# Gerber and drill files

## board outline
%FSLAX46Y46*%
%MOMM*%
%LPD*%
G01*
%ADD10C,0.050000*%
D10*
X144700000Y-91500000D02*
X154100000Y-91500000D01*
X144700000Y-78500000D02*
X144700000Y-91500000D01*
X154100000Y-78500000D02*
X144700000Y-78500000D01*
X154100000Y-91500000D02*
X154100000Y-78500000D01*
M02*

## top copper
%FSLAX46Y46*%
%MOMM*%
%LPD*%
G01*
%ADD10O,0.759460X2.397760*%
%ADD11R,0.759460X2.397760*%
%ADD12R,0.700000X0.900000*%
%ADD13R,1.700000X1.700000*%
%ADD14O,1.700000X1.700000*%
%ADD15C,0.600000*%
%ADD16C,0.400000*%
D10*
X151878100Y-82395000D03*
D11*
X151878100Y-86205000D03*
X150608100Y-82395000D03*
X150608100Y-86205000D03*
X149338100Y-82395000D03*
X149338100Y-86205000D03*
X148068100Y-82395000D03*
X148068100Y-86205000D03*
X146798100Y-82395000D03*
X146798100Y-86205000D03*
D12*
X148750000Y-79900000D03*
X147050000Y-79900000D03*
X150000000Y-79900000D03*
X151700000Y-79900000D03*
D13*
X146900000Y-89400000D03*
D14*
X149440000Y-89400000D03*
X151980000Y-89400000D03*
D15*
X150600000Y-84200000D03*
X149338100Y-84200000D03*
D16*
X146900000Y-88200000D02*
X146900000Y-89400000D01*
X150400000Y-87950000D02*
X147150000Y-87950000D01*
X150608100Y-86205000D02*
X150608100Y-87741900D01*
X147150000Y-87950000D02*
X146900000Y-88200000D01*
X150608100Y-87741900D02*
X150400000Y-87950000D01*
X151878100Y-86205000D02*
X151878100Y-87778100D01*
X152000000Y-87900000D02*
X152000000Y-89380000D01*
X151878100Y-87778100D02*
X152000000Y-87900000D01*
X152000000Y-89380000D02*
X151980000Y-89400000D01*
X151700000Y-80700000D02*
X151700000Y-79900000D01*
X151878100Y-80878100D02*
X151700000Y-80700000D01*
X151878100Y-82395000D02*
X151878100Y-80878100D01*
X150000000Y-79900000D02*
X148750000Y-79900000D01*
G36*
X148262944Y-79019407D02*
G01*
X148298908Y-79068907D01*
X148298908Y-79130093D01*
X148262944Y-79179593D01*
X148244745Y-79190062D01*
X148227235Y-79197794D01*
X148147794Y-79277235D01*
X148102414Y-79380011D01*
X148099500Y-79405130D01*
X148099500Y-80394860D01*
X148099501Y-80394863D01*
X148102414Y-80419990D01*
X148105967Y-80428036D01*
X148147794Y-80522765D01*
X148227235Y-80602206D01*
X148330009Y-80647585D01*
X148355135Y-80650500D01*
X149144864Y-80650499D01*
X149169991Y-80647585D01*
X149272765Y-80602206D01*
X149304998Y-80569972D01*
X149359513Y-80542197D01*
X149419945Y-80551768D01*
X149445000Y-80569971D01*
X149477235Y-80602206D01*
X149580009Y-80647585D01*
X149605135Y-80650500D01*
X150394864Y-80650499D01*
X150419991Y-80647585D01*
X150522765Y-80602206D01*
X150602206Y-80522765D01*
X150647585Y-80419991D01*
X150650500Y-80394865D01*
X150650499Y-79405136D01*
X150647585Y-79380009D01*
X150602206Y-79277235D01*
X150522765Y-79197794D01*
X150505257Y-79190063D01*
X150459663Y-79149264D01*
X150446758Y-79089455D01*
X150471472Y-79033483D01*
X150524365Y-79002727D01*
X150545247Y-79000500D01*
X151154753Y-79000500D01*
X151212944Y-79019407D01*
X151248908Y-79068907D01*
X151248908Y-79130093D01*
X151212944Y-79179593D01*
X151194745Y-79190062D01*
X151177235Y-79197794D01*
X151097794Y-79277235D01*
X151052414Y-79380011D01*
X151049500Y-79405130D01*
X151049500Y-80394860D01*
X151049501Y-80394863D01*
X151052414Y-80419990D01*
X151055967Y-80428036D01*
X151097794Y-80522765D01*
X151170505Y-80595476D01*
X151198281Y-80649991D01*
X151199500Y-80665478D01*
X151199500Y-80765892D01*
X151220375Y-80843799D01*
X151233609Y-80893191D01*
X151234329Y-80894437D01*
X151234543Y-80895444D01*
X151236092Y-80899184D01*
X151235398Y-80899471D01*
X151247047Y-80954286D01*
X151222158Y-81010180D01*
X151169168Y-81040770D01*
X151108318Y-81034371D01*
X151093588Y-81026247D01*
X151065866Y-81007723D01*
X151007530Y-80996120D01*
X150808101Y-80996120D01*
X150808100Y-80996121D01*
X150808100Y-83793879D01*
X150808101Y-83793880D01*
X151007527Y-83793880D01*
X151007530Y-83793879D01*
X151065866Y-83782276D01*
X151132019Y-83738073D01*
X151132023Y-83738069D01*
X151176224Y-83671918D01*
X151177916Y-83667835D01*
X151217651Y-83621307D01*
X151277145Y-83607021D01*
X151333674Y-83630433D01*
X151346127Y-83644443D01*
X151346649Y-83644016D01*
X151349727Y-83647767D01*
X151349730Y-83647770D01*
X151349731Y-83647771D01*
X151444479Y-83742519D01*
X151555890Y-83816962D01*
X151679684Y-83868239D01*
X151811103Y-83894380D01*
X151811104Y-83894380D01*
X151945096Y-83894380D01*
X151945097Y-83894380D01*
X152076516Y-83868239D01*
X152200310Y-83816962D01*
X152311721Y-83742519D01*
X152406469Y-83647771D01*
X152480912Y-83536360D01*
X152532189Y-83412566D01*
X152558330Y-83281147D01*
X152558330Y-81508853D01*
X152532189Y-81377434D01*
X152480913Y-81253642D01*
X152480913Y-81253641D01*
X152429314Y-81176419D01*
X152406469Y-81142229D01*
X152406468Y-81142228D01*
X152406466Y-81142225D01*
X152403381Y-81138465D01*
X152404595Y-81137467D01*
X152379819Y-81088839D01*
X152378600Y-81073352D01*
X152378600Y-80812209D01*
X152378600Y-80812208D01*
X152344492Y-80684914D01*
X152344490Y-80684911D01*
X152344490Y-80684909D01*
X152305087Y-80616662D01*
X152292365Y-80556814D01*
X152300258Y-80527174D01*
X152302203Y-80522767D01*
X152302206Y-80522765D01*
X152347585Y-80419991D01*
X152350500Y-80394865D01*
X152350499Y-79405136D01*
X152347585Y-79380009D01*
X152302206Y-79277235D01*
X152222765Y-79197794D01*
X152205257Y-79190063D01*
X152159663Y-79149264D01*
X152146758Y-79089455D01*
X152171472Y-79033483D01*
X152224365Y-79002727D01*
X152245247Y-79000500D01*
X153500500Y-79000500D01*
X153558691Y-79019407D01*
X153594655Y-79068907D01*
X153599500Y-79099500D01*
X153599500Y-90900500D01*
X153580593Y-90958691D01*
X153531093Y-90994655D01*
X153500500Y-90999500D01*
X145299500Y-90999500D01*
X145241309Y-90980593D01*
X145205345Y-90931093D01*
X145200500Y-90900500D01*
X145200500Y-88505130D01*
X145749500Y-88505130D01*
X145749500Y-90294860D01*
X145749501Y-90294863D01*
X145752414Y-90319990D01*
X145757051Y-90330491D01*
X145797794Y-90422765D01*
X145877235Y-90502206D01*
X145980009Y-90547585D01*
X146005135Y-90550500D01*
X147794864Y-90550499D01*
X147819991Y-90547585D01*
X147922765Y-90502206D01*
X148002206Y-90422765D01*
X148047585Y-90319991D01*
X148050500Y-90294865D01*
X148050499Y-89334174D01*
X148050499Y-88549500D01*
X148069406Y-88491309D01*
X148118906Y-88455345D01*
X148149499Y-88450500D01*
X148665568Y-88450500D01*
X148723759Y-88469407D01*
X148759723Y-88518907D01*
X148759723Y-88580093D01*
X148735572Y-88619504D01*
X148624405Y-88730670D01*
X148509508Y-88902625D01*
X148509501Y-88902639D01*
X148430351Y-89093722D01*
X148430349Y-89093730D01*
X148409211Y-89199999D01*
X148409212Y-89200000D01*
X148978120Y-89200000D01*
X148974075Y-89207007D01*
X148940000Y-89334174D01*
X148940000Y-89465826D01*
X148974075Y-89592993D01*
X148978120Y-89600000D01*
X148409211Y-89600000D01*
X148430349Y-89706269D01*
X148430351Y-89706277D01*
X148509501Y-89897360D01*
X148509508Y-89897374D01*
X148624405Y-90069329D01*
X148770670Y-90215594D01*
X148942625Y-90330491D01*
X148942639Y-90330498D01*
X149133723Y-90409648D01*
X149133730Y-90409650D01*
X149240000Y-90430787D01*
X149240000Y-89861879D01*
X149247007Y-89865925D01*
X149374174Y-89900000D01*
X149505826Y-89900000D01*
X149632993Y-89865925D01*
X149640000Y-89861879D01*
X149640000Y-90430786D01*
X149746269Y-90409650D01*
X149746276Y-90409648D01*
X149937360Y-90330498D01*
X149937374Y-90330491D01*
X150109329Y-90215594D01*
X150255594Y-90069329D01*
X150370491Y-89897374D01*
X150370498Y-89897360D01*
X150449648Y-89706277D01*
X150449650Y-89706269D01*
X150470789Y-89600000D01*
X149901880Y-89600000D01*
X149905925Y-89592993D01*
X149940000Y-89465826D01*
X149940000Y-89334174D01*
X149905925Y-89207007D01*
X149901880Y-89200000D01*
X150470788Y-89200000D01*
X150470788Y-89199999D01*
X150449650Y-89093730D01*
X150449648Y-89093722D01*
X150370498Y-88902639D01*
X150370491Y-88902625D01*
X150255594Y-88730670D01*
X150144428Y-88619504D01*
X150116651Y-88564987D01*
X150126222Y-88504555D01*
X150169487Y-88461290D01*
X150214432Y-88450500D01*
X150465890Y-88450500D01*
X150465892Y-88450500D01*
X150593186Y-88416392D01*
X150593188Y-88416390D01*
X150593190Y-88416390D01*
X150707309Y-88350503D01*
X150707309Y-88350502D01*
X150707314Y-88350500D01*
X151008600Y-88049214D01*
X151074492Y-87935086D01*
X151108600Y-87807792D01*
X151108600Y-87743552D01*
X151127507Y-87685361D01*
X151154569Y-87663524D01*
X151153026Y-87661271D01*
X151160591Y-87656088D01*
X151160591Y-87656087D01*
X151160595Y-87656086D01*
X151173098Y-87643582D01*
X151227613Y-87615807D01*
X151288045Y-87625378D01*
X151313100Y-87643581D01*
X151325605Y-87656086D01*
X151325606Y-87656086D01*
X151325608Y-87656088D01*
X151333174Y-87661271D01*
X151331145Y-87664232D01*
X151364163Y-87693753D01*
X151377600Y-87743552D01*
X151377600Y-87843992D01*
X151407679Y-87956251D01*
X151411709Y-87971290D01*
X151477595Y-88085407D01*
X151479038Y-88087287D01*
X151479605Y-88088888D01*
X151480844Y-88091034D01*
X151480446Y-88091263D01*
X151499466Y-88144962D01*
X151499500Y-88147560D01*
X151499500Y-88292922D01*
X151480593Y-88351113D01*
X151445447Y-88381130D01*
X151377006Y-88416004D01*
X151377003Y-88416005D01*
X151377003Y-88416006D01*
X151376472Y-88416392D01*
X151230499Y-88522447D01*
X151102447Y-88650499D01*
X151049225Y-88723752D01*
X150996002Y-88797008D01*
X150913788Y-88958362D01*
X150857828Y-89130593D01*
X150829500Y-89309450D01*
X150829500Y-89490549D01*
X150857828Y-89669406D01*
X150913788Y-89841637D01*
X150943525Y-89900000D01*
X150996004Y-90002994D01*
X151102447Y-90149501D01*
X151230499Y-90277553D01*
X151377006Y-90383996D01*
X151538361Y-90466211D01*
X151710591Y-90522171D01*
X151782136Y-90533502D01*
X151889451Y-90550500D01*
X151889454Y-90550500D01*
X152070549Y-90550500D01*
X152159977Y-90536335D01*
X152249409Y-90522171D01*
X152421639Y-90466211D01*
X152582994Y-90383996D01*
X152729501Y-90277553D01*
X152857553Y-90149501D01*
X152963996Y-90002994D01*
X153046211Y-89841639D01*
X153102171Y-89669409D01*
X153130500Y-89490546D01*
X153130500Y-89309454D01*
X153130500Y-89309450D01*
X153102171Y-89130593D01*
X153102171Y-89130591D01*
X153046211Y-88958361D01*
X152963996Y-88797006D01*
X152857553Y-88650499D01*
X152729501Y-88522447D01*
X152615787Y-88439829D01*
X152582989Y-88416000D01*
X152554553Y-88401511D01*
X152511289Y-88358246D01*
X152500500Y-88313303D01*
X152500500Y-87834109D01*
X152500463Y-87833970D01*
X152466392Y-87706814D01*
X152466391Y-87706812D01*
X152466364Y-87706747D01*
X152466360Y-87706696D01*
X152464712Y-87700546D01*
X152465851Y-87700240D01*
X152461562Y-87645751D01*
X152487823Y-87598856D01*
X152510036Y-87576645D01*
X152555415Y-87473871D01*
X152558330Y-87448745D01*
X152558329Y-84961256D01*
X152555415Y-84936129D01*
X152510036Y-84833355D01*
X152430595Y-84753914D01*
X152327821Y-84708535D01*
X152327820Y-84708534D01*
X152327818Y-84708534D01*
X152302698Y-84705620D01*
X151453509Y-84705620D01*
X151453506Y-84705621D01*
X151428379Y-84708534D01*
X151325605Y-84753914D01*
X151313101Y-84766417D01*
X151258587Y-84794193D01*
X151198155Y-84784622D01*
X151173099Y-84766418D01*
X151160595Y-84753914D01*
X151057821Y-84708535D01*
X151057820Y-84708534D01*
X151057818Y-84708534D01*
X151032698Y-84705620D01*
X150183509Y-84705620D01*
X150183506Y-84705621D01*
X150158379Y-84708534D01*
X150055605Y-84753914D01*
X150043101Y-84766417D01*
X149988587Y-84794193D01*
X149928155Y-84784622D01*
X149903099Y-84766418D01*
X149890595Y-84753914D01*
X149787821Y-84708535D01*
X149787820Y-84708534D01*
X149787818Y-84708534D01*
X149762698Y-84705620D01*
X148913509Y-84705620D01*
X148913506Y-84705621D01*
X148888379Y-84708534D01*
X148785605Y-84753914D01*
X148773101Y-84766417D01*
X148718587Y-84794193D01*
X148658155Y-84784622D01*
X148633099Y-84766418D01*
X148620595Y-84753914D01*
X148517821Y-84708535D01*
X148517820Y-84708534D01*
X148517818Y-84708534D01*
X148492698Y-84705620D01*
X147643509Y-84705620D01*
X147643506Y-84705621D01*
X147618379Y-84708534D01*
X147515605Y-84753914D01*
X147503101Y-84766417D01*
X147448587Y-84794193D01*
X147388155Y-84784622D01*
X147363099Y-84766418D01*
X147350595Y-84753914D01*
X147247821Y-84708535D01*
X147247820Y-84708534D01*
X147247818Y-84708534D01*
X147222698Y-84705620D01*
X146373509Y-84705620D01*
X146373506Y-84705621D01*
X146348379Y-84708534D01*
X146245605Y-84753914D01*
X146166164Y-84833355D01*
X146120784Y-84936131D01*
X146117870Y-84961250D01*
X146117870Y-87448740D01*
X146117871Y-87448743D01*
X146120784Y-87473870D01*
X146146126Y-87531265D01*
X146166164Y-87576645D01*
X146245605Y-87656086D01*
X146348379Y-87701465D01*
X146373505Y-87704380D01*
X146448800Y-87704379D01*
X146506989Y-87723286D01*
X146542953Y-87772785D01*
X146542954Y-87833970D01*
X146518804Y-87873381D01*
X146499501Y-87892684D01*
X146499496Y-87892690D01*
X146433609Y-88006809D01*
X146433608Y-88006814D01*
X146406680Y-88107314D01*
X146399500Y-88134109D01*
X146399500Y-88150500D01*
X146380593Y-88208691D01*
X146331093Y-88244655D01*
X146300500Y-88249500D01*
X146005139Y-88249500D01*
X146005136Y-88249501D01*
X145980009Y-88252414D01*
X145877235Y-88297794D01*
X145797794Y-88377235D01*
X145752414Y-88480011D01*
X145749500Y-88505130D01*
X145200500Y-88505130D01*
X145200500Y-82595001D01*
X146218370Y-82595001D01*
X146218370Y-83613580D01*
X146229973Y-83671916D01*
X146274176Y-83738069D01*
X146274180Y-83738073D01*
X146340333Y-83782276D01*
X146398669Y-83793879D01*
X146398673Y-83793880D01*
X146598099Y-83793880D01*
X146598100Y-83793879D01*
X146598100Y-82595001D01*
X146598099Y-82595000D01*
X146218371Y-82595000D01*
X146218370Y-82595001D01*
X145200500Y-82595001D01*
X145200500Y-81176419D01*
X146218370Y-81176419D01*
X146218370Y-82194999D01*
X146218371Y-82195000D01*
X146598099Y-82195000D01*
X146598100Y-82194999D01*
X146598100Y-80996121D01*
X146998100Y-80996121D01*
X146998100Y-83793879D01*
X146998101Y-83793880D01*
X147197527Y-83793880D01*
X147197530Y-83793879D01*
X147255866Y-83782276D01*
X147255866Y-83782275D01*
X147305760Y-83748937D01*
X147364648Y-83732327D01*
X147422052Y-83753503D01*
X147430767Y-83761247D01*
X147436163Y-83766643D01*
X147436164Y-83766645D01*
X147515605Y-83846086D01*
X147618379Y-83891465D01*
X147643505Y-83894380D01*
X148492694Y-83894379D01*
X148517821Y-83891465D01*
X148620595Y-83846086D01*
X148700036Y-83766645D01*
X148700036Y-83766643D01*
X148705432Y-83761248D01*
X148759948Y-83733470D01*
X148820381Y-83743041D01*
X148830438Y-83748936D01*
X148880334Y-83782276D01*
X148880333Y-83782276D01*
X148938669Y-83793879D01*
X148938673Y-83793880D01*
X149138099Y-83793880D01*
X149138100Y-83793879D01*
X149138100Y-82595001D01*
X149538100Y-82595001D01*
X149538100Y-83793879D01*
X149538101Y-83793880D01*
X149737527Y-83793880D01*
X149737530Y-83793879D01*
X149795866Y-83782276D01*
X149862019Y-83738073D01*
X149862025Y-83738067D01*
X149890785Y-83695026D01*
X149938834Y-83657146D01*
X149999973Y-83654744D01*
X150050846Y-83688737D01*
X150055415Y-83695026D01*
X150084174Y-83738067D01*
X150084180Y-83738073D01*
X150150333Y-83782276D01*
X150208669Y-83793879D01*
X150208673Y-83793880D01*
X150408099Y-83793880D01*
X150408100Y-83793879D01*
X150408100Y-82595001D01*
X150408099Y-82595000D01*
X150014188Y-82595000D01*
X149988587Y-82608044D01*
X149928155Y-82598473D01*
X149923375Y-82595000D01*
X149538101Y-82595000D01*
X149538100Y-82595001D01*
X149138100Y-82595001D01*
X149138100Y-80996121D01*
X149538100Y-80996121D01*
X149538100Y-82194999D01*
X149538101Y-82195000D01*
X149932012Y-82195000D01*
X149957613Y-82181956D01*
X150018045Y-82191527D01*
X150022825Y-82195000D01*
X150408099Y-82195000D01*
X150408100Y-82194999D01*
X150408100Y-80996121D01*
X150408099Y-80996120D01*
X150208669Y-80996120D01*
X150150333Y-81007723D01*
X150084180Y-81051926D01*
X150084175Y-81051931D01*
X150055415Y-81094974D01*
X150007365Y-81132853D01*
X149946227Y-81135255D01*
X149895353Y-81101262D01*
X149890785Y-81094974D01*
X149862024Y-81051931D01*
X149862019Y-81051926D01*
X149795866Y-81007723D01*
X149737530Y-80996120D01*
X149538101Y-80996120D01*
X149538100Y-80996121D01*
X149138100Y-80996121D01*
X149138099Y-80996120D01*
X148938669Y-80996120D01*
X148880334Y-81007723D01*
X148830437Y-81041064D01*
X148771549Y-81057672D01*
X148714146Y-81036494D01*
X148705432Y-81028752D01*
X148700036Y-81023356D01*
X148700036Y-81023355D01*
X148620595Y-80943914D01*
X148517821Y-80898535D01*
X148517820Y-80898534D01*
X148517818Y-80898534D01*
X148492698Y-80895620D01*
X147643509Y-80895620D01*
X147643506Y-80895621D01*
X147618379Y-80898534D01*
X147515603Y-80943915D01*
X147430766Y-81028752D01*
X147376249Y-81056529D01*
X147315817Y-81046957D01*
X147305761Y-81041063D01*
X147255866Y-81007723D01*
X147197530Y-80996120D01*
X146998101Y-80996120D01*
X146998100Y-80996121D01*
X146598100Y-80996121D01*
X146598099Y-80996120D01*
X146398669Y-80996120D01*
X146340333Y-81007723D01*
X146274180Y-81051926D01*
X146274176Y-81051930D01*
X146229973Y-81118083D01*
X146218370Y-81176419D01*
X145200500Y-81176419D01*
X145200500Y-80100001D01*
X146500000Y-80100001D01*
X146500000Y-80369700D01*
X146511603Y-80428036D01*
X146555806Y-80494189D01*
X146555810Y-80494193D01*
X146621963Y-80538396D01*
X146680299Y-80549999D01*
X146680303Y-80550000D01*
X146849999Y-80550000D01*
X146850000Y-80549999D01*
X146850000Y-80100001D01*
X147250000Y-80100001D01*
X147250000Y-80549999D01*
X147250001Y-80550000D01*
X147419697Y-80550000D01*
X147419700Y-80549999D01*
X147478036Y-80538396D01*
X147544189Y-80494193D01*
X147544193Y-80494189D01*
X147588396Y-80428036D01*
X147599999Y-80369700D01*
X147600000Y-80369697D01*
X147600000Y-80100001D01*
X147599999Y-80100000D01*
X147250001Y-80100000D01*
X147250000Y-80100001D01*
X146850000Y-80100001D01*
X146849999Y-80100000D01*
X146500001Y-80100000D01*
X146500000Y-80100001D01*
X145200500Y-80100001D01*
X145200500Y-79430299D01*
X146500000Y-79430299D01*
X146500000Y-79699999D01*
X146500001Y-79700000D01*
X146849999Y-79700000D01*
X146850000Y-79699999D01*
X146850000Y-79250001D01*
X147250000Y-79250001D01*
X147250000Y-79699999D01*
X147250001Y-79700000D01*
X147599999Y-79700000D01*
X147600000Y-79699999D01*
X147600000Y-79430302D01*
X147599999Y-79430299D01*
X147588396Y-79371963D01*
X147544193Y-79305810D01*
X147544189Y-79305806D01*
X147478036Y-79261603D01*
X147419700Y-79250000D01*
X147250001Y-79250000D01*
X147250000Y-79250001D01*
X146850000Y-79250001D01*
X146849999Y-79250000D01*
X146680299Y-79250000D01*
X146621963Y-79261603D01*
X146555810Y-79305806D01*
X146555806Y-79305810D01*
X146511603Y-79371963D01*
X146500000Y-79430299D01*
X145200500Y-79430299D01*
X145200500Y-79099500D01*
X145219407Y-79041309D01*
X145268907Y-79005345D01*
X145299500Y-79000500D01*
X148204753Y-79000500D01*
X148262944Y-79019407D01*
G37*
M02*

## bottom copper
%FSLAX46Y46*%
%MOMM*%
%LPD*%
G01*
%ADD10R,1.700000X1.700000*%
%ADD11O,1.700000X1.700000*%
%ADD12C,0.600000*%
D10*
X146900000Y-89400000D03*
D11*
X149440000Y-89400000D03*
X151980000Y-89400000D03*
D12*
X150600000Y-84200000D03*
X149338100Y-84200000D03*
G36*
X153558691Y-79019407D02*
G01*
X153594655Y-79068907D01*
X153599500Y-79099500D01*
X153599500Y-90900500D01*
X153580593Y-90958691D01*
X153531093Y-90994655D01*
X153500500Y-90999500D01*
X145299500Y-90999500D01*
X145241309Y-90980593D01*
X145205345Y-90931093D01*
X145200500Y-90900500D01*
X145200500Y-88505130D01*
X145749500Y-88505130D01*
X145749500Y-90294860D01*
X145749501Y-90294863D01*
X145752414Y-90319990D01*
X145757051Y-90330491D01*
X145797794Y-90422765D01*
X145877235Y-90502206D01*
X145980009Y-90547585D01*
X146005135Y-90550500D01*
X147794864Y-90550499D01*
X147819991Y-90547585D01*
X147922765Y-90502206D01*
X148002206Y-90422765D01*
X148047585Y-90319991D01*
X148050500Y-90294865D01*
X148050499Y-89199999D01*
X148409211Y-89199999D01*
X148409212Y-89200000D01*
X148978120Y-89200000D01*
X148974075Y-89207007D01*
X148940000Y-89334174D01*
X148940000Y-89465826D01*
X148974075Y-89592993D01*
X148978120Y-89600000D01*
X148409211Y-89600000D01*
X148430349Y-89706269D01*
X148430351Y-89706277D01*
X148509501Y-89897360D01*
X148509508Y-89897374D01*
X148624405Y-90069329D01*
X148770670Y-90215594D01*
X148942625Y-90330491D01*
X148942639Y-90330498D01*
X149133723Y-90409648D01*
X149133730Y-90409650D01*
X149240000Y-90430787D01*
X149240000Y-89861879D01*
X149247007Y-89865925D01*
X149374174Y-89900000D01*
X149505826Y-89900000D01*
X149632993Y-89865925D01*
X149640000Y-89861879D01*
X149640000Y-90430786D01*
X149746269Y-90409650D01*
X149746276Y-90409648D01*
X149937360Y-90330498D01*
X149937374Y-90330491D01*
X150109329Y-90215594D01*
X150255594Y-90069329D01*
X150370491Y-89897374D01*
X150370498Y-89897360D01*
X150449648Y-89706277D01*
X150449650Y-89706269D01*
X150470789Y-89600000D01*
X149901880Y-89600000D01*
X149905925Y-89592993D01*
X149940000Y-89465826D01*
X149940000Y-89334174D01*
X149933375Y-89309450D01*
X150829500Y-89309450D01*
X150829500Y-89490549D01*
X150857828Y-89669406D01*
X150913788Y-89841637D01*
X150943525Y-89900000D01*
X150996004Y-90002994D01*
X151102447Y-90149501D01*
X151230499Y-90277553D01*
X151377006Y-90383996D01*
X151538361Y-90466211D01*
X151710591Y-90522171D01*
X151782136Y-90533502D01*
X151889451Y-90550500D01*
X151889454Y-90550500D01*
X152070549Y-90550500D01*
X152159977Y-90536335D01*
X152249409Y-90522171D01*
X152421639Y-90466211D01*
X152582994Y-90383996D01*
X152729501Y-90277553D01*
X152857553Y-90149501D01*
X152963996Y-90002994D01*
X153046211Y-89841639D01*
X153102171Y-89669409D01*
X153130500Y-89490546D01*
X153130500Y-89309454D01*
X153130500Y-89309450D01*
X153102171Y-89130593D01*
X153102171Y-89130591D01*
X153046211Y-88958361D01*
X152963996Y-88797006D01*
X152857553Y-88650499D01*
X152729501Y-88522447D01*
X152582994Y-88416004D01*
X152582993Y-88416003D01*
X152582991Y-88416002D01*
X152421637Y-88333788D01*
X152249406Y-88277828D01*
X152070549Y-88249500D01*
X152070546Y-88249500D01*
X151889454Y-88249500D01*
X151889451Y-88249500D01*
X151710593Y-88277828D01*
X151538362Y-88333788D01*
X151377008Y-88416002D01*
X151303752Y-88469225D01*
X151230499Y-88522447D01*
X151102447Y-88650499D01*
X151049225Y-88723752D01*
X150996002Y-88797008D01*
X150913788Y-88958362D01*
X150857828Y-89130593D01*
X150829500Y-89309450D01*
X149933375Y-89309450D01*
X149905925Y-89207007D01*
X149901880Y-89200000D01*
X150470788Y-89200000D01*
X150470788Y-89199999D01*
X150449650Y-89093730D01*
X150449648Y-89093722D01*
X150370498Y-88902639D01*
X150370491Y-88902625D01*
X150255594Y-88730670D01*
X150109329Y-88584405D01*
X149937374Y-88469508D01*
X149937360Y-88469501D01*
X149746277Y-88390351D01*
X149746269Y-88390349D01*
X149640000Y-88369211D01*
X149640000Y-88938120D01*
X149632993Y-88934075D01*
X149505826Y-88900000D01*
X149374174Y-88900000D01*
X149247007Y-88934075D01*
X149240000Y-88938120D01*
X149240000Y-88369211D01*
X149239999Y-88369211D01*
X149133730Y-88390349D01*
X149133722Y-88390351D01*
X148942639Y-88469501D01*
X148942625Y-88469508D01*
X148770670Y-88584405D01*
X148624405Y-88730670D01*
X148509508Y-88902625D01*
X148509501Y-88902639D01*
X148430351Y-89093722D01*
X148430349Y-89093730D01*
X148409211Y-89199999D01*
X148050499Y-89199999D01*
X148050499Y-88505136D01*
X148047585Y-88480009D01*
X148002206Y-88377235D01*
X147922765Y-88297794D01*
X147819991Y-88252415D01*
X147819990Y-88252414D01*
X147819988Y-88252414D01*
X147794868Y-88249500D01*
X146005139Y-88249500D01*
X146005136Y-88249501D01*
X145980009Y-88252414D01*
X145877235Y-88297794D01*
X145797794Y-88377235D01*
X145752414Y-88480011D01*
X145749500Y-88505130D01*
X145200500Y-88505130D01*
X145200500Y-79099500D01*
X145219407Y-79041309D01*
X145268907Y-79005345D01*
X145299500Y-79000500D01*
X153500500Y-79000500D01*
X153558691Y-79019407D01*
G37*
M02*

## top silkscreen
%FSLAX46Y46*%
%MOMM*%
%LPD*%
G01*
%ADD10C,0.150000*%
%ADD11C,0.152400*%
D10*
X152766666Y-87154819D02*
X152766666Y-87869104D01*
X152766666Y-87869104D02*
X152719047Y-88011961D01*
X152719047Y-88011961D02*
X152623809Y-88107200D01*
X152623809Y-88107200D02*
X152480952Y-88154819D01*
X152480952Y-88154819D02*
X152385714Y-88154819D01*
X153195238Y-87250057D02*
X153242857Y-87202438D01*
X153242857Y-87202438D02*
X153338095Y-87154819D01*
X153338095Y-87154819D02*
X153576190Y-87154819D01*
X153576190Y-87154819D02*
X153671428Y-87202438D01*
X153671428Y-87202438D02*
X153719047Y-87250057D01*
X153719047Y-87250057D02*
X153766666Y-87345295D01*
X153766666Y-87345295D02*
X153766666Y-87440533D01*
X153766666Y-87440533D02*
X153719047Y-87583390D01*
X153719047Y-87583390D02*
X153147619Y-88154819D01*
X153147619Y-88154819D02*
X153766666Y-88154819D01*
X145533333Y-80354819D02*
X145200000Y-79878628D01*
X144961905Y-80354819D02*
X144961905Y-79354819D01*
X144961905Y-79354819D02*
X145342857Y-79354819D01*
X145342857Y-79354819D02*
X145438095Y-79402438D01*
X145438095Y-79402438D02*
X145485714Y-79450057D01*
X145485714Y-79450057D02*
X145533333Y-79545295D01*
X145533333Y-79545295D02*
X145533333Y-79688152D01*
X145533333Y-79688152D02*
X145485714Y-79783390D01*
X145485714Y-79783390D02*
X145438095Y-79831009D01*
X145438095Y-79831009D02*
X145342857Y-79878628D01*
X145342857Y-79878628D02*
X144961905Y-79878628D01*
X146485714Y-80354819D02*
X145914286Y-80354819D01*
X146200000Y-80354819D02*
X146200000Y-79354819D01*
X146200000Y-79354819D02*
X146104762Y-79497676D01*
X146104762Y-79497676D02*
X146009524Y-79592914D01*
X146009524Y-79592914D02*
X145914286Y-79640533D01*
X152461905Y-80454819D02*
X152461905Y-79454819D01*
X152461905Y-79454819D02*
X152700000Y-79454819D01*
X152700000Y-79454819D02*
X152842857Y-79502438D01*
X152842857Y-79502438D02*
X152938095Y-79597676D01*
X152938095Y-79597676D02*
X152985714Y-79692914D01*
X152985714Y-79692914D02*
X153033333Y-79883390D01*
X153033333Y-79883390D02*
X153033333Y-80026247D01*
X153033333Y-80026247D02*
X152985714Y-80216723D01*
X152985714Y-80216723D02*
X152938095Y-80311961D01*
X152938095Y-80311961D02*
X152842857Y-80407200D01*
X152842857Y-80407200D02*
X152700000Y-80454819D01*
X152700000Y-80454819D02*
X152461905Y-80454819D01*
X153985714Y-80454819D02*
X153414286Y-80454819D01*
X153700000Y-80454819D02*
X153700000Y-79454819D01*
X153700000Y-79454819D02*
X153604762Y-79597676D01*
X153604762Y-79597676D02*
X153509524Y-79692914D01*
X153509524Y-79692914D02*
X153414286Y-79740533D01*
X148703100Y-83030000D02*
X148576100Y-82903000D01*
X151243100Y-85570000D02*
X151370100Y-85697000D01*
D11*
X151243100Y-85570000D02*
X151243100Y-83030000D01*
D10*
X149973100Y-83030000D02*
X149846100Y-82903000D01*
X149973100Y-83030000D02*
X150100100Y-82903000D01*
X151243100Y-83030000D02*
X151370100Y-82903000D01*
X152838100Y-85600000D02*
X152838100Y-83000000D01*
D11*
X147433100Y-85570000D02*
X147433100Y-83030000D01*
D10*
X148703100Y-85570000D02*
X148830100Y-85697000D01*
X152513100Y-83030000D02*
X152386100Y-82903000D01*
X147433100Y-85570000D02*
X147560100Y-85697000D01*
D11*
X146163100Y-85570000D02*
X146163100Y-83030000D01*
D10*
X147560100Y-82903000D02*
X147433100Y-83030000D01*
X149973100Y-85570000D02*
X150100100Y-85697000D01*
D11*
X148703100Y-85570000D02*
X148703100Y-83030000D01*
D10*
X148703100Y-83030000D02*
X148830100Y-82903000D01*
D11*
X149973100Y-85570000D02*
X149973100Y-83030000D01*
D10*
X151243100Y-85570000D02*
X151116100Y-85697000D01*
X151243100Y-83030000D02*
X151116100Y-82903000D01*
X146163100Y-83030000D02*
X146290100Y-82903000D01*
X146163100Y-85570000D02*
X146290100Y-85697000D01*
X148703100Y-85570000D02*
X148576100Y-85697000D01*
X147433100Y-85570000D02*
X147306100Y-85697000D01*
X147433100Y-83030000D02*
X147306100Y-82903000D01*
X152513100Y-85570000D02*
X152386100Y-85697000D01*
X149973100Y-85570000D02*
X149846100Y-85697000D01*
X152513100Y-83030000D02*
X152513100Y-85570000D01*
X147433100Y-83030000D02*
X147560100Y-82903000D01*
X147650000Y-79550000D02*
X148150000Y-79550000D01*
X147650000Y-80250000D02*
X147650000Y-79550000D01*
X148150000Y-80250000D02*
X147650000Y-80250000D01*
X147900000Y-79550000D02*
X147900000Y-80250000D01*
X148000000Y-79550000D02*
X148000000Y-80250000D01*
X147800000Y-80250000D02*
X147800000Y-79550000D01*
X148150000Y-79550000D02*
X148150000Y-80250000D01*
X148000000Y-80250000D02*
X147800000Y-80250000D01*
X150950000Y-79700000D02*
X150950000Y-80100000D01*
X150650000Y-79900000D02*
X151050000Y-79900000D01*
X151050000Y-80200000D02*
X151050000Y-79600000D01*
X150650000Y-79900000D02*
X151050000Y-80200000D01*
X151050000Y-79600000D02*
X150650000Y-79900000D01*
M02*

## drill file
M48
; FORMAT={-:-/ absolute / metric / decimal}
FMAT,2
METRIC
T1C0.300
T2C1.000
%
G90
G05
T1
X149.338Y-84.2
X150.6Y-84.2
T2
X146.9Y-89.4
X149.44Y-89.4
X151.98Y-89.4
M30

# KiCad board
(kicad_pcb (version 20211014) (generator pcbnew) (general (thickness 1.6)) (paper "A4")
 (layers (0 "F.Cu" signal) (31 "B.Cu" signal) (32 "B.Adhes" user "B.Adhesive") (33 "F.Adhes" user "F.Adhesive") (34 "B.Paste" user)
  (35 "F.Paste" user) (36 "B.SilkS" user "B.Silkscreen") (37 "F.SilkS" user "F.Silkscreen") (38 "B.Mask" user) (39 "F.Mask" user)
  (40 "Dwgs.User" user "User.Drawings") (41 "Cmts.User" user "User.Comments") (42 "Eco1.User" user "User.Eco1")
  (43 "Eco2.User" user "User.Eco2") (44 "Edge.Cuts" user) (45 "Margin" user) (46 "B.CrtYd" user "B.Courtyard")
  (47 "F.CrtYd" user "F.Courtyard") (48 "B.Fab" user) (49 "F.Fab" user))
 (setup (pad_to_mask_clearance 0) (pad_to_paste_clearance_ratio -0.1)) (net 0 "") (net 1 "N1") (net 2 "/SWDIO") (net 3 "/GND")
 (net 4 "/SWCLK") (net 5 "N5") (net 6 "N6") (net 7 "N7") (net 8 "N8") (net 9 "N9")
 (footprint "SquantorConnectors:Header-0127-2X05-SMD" (layer "F.Cu") (at 149.3381 84.3 180)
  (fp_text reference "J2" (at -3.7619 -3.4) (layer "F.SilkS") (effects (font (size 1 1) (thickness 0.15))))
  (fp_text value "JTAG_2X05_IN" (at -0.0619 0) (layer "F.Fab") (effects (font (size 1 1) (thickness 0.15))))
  (fp_line (start 0.635 1.27) (end 0.762 1.397) (layer "F.SilkS") (width 0.15))
  (fp_line (start -1.905 -1.27) (end -2.032 -1.397) (layer "F.SilkS") (width 0.15))
  (fp_line (start -1.905 -1.27) (end -1.905 1.27) (layer "F.SilkS") (width 0.1524))
  (fp_line (start -0.635 1.27) (end -0.508 1.397) (layer "F.SilkS") (width 0.15))
  (fp_line (start -0.635 1.27) (end -0.762 1.397) (layer "F.SilkS") (width 0.15))
  (fp_line (start -1.905 1.27) (end -2.032 1.397) (layer "F.SilkS") (width 0.15))
  (fp_line (start -3.5 -1.3) (end -3.5 1.3) (layer "F.SilkS") (width 0.15))
  (fp_line (start 1.905 -1.27) (end 1.905 1.27) (layer "F.SilkS") (width 0.1524))
  (fp_line (start 0.635 -1.27) (end 0.508 -1.397) (layer "F.SilkS") (width 0.15))
  (fp_line (start -3.175 1.27) (end -3.048 1.397) (layer "F.SilkS") (width 0.15))
  (fp_line (start 1.905 -1.27) (end 1.778 -1.397) (layer "F.SilkS") (width 0.15))
  (fp_line (start 3.175 -1.27) (end 3.175 1.27) (layer "F.SilkS") (width 0.1524))
  (fp_line (start 1.778 1.397) (end 1.905 1.27) (layer "F.SilkS") (width 0.15))
  (fp_line (start -0.635 -1.27) (end -0.762 -1.397) (layer "F.SilkS") (width 0.15))
  (fp_line (start 0.635 -1.27) (end 0.635 1.27) (layer "F.SilkS") (width 0.1524))
  (fp_line (start 0.635 1.27) (end 0.508 1.397) (layer "F.SilkS") (width 0.15))
  (fp_line (start -0.635 -1.27) (end -0.635 1.27) (layer "F.SilkS") (width 0.1524))
  (fp_line (start -1.905 -1.27) (end -1.778 -1.397) (layer "F.SilkS") (width 0.15))
  (fp_line (start -1.905 1.27) (end -1.778 1.397) (layer "F.SilkS") (width 0.15))
  (fp_line (start 3.175 1.27) (end 3.048 1.397) (layer "F.SilkS") (width 0.15))
  (fp_line (start 3.175 -1.27) (end 3.048 -1.397) (layer "F.SilkS") (width 0.15))
  (fp_line (start 0.635 -1.27) (end 0.762 -1.397) (layer "F.SilkS") (width 0.15))
  (fp_line (start 1.905 -1.27) (end 2.032 -1.397) (layer "F.SilkS") (width 0.15))
  (fp_line (start 1.905 1.27) (end 2.032 1.397) (layer "F.SilkS") (width 0.15))
  (fp_line (start -3.175 -1.27) (end -3.048 -1.397) (layer "F.SilkS") (width 0.15))
  (fp_line (start -0.635 -1.27) (end -0.508 -1.397) (layer "F.SilkS") (width 0.15))
  (fp_line (start -3.175 1.27) (end -3.175 -1.27) (layer "F.SilkS") (width 0.15))
  (fp_line (start 1.905 1.27) (end 1.778 1.397) (layer "F.SilkS") (width 0.15))
  (pad "1" smd oval (at -2.54 1.905 270) (size 2.39776 0.75946) (layers "F.Cu" "F.Paste" "F.Mask") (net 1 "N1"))
  (pad "2" smd rect (at -2.54 -1.905 270) (size 2.39776 0.75946) (layers "F.Cu" "F.Paste" "F.Mask") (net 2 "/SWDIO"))
  (pad "3" smd rect (at -1.27 1.905 270) (size 2.39776 0.75946) (layers "F.Cu" "F.Paste" "F.Mask") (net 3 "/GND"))
  (pad "4" smd rect (at -1.27 -1.905 270) (size 2.39776 0.75946) (layers "F.Cu" "F.Paste" "F.Mask") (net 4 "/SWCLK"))
  (pad "5" smd rect (at 0 1.905 270) (size 2.39776 0.75946) (layers "F.Cu" "F.Paste" "F.Mask") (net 3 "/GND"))
  (pad "6" smd rect (at 0 -1.905 270) (size 2.39776 0.75946) (layers "F.Cu" "F.Paste" "F.Mask") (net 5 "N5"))
  (pad "7" smd rect (at 1.27 1.905 270) (size 2.39776 0.75946) (layers "F.Cu" "F.Paste" "F.Mask") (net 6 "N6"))
  (pad "8" smd rect (at 1.27 -1.905 270) (size 2.39776 0.75946) (layers "F.Cu" "F.Paste" "F.Mask") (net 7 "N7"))
  (pad "9" smd rect (at 2.54 1.905 270) (size 2.39776 0.75946) (layers "F.Cu" "F.Paste" "F.Mask") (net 3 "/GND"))
  (pad "10" smd rect (at 2.54 -1.905 270) (size 2.39776 0.75946) (layers "F.Cu" "F.Paste" "F.Mask") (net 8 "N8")))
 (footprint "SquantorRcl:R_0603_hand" (layer "F.Cu") (at 147.9 79.9 180)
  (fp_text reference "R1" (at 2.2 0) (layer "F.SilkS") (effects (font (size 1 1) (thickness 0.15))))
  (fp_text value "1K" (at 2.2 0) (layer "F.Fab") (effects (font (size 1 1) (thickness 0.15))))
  (fp_line (start 0.25 0.35) (end -0.25 0.35) (layer "F.SilkS") (width 0.15))
  (fp_line (start 0.25 -0.35) (end 0.25 0.35) (layer "F.SilkS") (width 0.15))
  (fp_line (start -0.25 -0.35) (end 0.25 -0.35) (layer "F.SilkS") (width 0.15))
  (fp_line (start 0 0.35) (end 0 -0.35) (layer "F.SilkS") (width 0.15))
  (fp_line (start -0.1 0.35) (end -0.1 -0.35) (layer "F.SilkS") (width 0.15))
  (fp_line (start 0.1 -0.35) (end 0.1 0.35) (layer "F.SilkS") (width 0.15))
  (fp_line (start -0.25 0.35) (end -0.25 -0.35) (layer "F.SilkS") (width 0.15))
  (fp_line (start -0.1 -0.35) (end 0.1 -0.35) (layer "F.SilkS") (width 0.15))
  (pad "1" smd rect (at -0.85 0 180) (size 0.7 0.9) (layers "F.Cu" "F.Paste" "F.Mask") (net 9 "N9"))
  (pad "2" smd rect (at 0.85 0 180) (size 0.7 0.9) (layers "F.Cu" "F.Paste" "F.Mask") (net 3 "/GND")))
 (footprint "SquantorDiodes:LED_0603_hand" (layer "F.Cu") (at 150.85 79.9)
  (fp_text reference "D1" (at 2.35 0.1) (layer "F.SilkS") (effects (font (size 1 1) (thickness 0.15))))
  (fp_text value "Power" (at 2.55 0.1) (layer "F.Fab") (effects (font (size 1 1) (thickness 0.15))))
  (fp_line (start 0.1 -0.2) (end 0.1 0.2) (layer "F.SilkS") (width 0.15))
  (fp_line (start -0.2 0) (end 0.2 0) (layer "F.SilkS") (width 0.15))
  (fp_line (start 0.2 0.3) (end 0.2 -0.3) (layer "F.SilkS") (width 0.15))
  (fp_line (start -0.2 0) (end 0.2 0.3) (layer "F.SilkS") (width 0.15))
  (fp_line (start 0.2 -0.3) (end -0.2 0) (layer "F.SilkS") (width 0.15))
  (pad "1" smd rect (at -0.85 0) (size 0.7 0.9) (layers "F.Cu" "F.Paste" "F.Mask") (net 9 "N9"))
  (pad "2" smd rect (at 0.85 0) (size 0.7 0.9) (layers "F.Cu" "F.Paste" "F.Mask") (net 1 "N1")))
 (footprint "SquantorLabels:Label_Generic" (layer "B.Cu") (at 150.2 85.8 180)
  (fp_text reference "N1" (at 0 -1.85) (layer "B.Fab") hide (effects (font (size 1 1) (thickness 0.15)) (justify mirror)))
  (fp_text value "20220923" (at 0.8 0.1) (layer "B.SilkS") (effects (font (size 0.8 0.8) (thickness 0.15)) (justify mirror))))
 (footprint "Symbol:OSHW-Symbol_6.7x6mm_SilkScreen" (layer "B.Cu") (at 149.4 81.9 180)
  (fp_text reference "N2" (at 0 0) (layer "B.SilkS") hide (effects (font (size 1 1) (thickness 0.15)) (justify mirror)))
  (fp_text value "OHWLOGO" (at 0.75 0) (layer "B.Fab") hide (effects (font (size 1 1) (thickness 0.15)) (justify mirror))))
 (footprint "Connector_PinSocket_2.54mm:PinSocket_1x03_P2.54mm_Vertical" (layer "B.Cu") (at 146.9 89.4 -90)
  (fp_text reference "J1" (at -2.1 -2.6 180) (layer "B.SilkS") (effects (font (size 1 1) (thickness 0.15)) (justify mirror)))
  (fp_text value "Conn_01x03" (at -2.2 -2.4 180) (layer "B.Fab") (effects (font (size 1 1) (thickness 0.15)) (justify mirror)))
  (pad "1" thru_hole rect (at 0 0 270) (size 1.7 1.7) (drill 1) (layers *.Cu *.Mask) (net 4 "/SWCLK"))
  (pad "2" thru_hole oval (at 0 -2.54 270) (size 1.7 1.7) (drill 1) (layers *.Cu *.Mask) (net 3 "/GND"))
  (pad "3" thru_hole oval (at 0 -5.08 270) (size 1.7 1.7) (drill 1) (layers *.Cu *.Mask) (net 2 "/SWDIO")))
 (gr_line (start 144.7 91.5) (end 154.1 91.5) (layer "Edge.Cuts") (width 0.05))
 (gr_line (start 144.7 78.5) (end 144.7 91.5) (layer "Edge.Cuts") (width 0.05))
 (gr_line (start 154.1 78.5) (end 144.7 78.5) (layer "Edge.Cuts") (width 0.05))
 (gr_line (start 154.1 91.5) (end 154.1 78.5) (layer "Edge.Cuts") (width 0.05))
 (segment (start 146.9 88.2) (end 146.9 89.4) (width 0.4) (layer "F.Cu") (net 4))
 (segment (start 150.4 87.95) (end 147.15 87.95) (width 0.4) (layer "F.Cu") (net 4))
 (segment (start 150.6081 86.205) (end 150.6081 87.7419) (width 0.4) (layer "F.Cu") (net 4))
 (segment (start 147.15 87.95) (end 146.9 88.2) (width 0.4) (layer "F.Cu") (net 4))
 (segment (start 150.6081 87.7419) (end 150.4 87.95) (width 0.4) (layer "F.Cu") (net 4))
 (via (at 150.6 84.2) (size 0.6) (drill 0.3) (layers "F.Cu" "B.Cu") (free) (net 3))
 (via (at 149.3381 84.2) (size 0.6) (drill 0.3) (layers "F.Cu" "B.Cu") (free) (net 3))
 (segment (start 151.8781 86.205) (end 151.8781 87.7781) (width 0.4) (layer "F.Cu") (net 2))
 (segment (start 152 87.9) (end 152 89.38) (width 0.4) (layer "F.Cu") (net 2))
 (segment (start 151.8781 87.7781) (end 152 87.9) (width 0.4) (layer "F.Cu") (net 2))
 (segment (start 152 89.38) (end 151.98 89.4) (width 0.4) (layer "F.Cu") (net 2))
 (segment (start 151.7 80.7) (end 151.7 79.9) (width 0.4) (layer "F.Cu") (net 1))
 (segment (start 151.8781 80.8781) (end 151.7 80.7) (width 0.4) (layer "F.Cu") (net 1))
 (segment (start 151.8781 82.395) (end 151.8781 80.8781) (width 0.4) (layer "F.Cu") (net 1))
 (segment (start 150 79.9) (end 148.75 79.9) (width 0.4) (layer "F.Cu") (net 9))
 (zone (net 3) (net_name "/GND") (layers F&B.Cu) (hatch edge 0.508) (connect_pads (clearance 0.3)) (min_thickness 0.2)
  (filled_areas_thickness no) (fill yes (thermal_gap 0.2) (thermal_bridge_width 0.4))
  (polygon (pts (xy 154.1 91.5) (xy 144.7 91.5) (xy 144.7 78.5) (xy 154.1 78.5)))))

